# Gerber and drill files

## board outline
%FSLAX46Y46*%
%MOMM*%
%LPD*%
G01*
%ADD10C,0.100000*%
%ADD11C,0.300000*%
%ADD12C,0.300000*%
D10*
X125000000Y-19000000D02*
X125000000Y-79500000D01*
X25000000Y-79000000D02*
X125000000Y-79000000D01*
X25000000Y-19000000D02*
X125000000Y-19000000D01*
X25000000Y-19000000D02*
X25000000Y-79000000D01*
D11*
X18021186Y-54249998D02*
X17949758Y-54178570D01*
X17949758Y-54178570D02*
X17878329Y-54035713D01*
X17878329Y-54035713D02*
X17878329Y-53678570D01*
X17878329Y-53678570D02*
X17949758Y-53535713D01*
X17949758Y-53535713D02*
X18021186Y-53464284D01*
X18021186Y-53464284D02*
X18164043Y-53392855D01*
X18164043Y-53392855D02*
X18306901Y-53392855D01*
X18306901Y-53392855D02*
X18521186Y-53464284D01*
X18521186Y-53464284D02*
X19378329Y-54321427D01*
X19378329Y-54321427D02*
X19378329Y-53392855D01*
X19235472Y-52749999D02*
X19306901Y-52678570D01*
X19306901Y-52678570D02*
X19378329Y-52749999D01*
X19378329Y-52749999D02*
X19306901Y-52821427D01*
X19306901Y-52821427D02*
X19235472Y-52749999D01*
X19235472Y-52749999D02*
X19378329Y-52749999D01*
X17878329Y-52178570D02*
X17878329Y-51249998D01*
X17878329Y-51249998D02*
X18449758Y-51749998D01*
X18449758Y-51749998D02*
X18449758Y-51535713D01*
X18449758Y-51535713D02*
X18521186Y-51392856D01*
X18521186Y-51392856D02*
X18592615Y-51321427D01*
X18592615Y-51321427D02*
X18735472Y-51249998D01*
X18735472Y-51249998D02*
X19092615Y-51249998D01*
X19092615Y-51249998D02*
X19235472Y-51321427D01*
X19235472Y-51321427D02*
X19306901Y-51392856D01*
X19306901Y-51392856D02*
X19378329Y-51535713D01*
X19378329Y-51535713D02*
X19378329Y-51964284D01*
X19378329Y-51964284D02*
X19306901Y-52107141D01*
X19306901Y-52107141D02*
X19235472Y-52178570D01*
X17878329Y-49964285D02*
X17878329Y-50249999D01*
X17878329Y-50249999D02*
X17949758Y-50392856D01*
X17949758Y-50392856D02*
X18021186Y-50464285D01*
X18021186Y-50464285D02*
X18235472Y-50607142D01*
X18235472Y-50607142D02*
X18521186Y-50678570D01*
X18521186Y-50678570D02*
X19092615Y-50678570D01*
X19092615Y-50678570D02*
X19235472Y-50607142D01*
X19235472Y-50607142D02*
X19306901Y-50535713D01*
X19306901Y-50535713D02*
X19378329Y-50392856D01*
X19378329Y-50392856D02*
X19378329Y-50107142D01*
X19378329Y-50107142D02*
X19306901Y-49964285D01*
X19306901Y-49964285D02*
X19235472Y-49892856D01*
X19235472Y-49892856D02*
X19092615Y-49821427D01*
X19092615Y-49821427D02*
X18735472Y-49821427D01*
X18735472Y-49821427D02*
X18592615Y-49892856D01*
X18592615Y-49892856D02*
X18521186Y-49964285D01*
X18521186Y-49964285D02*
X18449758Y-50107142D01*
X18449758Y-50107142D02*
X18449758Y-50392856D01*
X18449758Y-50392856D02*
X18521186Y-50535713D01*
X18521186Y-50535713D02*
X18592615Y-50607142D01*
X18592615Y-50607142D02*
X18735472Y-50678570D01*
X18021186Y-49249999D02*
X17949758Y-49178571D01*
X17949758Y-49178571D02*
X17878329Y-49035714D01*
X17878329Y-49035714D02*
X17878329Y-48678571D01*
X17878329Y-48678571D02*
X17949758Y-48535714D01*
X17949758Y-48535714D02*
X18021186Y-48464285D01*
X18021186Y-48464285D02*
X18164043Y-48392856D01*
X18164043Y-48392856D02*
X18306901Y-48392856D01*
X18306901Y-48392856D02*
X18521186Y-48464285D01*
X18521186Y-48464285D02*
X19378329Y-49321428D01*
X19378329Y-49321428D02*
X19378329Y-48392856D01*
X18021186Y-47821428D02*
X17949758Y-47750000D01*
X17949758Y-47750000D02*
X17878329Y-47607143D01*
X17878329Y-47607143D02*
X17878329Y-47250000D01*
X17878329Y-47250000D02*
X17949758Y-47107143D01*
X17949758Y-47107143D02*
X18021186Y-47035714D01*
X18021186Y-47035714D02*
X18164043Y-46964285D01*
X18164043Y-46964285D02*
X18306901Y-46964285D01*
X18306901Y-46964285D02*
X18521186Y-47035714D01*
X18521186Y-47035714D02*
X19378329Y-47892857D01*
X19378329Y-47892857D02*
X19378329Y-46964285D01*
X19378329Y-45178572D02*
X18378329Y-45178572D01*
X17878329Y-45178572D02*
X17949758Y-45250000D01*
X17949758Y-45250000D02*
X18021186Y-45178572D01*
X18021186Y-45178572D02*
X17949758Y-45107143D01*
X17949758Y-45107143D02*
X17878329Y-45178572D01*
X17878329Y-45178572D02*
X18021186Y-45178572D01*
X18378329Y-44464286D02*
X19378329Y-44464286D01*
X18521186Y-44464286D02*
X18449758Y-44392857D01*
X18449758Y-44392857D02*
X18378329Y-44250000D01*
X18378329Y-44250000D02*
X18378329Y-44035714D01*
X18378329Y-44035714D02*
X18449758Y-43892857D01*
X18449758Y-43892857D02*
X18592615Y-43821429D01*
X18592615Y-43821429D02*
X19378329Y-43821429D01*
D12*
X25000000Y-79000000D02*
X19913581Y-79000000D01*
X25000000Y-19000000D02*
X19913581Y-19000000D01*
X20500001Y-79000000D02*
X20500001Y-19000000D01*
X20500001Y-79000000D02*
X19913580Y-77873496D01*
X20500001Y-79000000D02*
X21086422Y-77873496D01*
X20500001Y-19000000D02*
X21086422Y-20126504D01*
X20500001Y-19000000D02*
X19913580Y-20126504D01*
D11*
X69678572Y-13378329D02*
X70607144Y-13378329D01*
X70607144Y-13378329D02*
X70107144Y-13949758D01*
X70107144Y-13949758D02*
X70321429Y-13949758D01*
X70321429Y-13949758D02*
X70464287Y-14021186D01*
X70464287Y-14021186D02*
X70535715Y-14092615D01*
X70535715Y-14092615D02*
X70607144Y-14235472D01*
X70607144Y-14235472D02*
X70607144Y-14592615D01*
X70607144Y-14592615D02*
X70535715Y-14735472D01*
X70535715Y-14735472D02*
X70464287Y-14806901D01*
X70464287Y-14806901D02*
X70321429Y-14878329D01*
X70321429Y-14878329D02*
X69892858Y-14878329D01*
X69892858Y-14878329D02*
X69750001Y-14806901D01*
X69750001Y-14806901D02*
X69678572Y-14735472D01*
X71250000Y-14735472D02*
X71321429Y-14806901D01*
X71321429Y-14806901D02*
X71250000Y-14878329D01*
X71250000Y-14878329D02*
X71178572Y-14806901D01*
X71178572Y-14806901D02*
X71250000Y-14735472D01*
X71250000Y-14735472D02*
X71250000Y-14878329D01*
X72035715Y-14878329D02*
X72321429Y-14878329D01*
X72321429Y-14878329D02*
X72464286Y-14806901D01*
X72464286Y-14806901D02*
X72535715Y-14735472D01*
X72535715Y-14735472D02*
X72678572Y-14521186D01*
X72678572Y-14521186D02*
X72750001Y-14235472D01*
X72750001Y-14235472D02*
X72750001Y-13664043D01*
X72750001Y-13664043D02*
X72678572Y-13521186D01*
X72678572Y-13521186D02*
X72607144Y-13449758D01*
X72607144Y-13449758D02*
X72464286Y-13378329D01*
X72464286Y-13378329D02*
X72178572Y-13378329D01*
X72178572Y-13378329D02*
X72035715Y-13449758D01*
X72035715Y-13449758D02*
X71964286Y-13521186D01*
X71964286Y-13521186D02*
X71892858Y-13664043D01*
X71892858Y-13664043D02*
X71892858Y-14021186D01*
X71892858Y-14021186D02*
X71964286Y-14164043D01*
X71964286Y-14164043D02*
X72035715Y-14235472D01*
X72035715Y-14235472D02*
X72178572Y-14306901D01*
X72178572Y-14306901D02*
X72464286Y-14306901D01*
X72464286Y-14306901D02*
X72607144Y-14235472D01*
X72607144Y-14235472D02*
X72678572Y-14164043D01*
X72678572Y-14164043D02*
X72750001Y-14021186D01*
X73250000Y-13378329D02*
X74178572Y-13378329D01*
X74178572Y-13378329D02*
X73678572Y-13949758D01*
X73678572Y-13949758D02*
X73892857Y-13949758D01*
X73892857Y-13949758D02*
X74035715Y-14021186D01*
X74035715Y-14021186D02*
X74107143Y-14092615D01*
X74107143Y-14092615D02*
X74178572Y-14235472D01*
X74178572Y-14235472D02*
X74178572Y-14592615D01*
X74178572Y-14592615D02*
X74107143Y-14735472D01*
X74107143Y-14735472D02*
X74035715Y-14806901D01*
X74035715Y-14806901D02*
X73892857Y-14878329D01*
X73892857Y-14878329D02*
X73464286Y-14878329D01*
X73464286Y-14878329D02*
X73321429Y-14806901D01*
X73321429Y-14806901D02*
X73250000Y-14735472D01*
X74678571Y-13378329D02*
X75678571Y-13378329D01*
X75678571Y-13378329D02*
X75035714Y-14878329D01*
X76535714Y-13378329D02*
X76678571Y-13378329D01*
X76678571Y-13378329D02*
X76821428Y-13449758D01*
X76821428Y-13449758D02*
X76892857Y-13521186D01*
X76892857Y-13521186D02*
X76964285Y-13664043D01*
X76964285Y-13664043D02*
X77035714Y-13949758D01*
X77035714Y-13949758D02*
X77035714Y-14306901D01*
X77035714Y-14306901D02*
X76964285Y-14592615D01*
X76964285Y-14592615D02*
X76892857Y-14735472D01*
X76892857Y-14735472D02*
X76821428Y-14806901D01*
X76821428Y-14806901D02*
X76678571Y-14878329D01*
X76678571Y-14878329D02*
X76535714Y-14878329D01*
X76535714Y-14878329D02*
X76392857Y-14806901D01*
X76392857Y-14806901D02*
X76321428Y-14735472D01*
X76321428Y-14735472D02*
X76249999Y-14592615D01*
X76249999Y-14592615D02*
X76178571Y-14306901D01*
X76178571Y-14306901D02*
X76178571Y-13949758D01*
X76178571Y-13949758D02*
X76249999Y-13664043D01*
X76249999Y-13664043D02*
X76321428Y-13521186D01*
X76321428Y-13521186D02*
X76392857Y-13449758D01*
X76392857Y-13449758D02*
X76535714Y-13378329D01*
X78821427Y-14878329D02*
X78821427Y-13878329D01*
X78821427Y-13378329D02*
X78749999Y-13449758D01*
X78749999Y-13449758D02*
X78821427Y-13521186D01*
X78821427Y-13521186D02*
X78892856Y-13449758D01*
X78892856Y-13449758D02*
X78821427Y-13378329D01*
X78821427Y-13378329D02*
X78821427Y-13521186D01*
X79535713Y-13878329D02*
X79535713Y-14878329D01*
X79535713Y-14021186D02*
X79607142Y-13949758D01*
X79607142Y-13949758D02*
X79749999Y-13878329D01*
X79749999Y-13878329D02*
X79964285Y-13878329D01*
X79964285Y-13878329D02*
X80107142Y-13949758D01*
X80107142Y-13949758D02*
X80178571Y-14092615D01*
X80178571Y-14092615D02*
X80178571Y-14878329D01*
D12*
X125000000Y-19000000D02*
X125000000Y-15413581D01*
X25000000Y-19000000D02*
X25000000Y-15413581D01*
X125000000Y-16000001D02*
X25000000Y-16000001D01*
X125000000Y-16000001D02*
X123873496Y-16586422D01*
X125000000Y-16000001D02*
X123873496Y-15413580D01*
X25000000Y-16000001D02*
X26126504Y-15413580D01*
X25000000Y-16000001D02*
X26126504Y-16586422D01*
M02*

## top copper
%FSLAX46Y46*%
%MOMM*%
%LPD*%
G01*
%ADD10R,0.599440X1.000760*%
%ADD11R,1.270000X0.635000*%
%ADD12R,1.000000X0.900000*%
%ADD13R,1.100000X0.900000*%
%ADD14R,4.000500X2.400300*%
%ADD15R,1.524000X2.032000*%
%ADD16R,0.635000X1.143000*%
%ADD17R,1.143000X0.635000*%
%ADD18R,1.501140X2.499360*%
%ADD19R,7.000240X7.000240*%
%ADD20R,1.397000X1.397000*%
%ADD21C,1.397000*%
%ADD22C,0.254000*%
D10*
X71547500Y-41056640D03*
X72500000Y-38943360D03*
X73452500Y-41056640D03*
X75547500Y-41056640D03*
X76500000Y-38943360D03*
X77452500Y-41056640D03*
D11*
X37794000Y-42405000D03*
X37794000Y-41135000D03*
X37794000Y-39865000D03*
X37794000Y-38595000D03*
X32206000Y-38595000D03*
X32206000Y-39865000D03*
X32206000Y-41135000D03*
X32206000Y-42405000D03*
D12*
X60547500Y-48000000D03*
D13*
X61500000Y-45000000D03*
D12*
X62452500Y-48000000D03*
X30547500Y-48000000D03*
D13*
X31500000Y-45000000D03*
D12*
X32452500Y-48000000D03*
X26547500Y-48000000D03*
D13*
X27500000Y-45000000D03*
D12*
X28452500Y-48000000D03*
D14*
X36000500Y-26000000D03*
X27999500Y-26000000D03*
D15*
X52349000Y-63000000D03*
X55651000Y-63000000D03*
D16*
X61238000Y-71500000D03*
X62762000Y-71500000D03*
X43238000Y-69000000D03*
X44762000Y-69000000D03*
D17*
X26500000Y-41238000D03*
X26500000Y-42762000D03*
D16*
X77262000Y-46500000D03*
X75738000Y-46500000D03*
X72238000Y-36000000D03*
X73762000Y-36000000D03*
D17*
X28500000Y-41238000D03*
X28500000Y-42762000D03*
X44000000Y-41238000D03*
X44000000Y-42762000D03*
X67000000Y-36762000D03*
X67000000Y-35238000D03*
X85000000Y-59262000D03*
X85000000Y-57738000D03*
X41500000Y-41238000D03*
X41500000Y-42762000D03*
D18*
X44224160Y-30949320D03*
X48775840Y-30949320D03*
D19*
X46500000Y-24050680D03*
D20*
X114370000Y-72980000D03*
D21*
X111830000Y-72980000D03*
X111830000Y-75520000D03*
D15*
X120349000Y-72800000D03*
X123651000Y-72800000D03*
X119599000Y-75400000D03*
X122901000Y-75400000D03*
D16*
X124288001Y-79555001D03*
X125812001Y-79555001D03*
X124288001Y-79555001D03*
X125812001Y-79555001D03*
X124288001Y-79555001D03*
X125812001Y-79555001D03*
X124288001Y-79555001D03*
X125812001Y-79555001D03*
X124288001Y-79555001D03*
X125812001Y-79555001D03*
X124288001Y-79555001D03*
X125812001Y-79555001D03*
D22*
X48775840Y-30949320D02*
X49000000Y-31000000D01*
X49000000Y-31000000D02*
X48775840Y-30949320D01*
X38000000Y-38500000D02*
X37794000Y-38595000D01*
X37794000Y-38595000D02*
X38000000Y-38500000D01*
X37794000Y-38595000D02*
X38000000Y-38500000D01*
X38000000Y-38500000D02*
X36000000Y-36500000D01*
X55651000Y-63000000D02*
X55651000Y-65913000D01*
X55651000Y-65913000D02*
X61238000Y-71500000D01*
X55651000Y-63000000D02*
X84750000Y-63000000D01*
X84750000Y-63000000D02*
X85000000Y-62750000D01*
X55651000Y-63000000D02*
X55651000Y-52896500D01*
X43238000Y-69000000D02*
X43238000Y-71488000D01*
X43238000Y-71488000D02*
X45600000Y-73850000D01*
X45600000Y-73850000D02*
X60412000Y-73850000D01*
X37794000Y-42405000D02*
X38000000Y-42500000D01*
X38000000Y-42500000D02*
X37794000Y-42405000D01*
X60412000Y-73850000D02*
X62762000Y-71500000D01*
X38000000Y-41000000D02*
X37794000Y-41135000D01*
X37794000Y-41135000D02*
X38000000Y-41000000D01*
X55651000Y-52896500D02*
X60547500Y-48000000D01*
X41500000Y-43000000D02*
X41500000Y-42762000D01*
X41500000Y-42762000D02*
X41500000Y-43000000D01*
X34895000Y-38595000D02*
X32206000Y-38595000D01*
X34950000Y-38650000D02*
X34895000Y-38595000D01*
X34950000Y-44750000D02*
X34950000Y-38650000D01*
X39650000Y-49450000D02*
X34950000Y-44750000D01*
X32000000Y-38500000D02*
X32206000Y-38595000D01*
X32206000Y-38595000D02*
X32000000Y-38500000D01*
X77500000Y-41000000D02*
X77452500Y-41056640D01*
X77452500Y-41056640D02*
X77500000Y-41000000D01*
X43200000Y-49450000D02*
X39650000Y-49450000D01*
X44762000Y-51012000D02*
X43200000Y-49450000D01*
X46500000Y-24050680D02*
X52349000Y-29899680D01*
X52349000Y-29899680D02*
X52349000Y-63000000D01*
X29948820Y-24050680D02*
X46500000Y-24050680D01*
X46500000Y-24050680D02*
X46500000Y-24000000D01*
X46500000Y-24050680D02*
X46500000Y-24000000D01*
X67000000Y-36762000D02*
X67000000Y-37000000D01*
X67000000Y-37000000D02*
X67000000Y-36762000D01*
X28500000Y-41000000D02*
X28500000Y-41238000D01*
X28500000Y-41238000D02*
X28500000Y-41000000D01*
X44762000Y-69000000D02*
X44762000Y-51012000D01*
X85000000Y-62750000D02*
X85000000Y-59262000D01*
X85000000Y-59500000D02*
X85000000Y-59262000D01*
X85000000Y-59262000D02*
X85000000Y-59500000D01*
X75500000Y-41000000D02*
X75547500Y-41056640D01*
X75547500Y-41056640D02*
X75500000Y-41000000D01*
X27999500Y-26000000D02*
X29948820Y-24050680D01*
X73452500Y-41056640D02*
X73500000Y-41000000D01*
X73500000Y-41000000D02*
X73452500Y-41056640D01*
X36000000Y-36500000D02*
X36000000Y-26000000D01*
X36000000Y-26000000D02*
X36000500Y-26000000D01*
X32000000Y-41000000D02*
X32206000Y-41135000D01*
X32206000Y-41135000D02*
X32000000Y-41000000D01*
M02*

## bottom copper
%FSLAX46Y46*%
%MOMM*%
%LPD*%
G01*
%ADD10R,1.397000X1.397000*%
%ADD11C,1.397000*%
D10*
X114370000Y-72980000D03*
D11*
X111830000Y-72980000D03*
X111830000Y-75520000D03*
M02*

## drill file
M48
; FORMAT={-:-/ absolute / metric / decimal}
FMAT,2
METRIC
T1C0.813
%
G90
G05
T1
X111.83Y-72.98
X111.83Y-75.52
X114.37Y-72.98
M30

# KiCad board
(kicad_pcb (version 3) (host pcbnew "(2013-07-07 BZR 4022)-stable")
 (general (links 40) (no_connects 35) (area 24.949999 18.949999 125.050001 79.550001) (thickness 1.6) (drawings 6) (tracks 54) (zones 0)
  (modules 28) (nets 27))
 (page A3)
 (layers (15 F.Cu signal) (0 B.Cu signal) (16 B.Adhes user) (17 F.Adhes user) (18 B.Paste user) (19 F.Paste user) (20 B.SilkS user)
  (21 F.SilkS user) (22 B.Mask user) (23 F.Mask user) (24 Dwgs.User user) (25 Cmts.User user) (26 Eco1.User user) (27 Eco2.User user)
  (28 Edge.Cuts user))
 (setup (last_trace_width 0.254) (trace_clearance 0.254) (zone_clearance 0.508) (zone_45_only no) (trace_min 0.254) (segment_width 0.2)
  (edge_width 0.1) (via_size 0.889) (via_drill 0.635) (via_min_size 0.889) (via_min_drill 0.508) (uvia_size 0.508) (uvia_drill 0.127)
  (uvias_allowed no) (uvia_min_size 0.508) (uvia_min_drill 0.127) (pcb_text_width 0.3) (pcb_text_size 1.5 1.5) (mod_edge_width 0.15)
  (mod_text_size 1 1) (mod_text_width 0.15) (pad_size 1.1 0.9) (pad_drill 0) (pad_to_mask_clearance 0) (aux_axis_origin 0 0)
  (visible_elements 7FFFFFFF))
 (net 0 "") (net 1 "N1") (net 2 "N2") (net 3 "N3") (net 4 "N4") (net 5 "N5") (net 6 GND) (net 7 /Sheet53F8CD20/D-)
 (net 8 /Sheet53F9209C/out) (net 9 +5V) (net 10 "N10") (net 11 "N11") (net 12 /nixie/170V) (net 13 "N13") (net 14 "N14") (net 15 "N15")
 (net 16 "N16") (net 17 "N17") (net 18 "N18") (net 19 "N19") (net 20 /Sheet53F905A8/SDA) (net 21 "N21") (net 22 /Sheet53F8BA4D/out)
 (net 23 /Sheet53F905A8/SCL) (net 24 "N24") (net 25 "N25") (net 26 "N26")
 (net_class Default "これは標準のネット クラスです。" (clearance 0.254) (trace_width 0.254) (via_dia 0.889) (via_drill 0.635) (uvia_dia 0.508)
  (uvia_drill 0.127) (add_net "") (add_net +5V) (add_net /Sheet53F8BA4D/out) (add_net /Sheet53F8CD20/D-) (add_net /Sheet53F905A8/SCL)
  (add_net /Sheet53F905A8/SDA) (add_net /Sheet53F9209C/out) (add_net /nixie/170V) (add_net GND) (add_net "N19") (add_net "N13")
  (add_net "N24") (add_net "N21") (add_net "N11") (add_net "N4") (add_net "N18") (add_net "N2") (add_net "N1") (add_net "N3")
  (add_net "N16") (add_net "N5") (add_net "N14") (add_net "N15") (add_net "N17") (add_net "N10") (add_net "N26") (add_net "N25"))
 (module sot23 (layer F.Cu) (at 72.5 40)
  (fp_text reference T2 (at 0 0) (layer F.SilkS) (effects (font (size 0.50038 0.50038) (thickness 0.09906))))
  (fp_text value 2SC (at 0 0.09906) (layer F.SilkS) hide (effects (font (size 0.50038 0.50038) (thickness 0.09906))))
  (pad 1 smd rect (at -0.9525 1.05664) (size 0.59944 1.00076) (layers F.Cu F.Paste F.Mask) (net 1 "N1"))
  (pad 2 smd rect (at 0 -1.05664) (size 0.59944 1.00076) (layers F.Cu F.Paste F.Mask) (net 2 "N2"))
  (pad 3 smd rect (at 0.9525 1.05664) (size 0.59944 1.00076) (layers F.Cu F.Paste F.Mask) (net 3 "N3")))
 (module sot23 (layer F.Cu) (at 76.5 40)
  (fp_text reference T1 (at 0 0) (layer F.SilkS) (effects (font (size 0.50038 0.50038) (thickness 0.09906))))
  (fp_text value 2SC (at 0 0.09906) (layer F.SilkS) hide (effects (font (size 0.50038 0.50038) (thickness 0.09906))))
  (pad 1 smd rect (at -0.9525 1.05664) (size 0.59944 1.00076) (layers F.Cu F.Paste F.Mask) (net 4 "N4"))
  (pad 2 smd rect (at 0 -1.05664) (size 0.59944 1.00076) (layers F.Cu F.Paste F.Mask) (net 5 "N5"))
  (pad 3 smd rect (at 0.9525 1.05664) (size 0.59944 1.00076) (layers F.Cu F.Paste F.Mask) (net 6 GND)))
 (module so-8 (layer F.Cu) (at 35 40.5 90)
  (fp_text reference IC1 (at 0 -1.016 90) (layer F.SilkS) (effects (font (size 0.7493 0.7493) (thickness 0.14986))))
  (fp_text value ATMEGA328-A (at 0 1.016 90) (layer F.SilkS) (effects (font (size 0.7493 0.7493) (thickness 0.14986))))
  (pad 1 smd rect (at -1.905 2.794 90) (size 0.635 1.27) (layers F.Cu F.Paste F.Mask) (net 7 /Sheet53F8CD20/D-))
  (pad 2 smd rect (at -0.635 2.794 90) (size 0.635 1.27) (layers F.Cu F.Paste F.Mask) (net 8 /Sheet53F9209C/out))
  (pad 3 smd rect (at 0.635 2.794 90) (size 0.635 1.27) (layers F.Cu F.Paste F.Mask) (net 6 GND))
  (pad 4 smd rect (at 1.905 2.794 90) (size 0.635 1.27) (layers F.Cu F.Paste F.Mask) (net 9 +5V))
  (pad 5 smd rect (at 1.905 -2.794 90) (size 0.635 1.27) (layers F.Cu F.Paste F.Mask) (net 6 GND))
  (pad 6 smd rect (at 0.635 -2.794 90) (size 0.635 1.27) (layers F.Cu F.Paste F.Mask) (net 9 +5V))
  (pad 7 smd rect (at -0.635 -2.794 90) (size 0.635 1.27) (layers F.Cu F.Paste F.Mask) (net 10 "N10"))
  (pad 8 smd rect (at -1.905 -2.794 90) (size 0.635 1.27) (layers F.Cu F.Paste F.Mask) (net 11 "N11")))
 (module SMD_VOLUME (layer F.Cu) (at 61.5 46.5)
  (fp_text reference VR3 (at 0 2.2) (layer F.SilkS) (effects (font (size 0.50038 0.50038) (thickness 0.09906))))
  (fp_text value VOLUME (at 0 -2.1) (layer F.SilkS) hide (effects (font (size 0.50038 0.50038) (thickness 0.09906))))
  (pad 1 smd rect (at -0.9525 1.5) (size 1 0.9) (layers F.Cu F.Paste F.Mask) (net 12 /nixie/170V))
  (pad 2 smd rect (at 0 -1.5) (size 1.1 0.9) (layers F.Cu F.Paste F.Mask) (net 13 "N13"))
  (pad 3 smd rect (at 0.9525 1.5) (size 1 0.9) (layers F.Cu F.Paste F.Mask) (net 13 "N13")))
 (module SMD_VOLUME (layer F.Cu) (at 31.5 46.5)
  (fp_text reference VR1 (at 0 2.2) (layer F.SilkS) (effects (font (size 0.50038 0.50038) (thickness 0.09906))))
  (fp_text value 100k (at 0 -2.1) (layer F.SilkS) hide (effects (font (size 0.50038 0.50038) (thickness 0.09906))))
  (pad 1 smd rect (at -0.9525 1.5) (size 1 0.9) (layers F.Cu F.Paste F.Mask) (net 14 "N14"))
  (pad 2 smd rect (at 0 -1.5) (size 1.1 0.9) (layers F.Cu F.Paste F.Mask) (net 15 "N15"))
  (pad 3 smd rect (at 0.9525 1.5) (size 1 0.9) (layers F.Cu F.Paste F.Mask) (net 15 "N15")))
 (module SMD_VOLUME (layer F.Cu) (at 27.5 46.5)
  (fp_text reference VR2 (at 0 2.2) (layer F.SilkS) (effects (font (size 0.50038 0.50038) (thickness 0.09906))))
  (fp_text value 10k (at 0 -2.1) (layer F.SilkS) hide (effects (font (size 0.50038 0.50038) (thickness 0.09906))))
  (pad 1 smd rect (at -0.9525 1.5) (size 1 0.9) (layers F.Cu F.Paste F.Mask) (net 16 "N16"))
  (pad 2 smd rect (at 0 -1.5) (size 1.1 0.9) (layers F.Cu F.Paste F.Mask) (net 6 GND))
  (pad 3 smd rect (at 0.9525 1.5) (size 1 0.9) (layers F.Cu F.Paste F.Mask) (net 6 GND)))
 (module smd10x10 (layer F.Cu) (at 32 26)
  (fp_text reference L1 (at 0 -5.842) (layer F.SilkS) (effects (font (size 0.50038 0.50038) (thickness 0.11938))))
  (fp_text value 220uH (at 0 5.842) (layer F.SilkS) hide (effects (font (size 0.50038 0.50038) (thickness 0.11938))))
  (pad 1 smd rect (at 4.0005 0) (size 4.0005 2.4003) (layers F.Cu F.Paste F.Mask) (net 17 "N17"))
  (pad 2 smd rect (at -4.0005 0) (size 4.0005 2.4003) (layers F.Cu F.Paste F.Mask) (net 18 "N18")))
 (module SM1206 (layer F.Cu) (at 54 63)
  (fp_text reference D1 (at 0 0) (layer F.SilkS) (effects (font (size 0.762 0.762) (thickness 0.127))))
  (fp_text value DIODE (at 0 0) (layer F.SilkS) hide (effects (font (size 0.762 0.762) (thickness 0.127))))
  (pad 1 smd rect (at -1.651 0) (size 1.524 2.032) (layers F.Cu F.Paste F.Mask) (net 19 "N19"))
  (pad 2 smd rect (at 1.651 0) (size 1.524 2.032) (layers F.Cu F.Paste F.Mask) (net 9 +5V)))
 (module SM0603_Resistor (layer F.Cu) (at 62 71.5)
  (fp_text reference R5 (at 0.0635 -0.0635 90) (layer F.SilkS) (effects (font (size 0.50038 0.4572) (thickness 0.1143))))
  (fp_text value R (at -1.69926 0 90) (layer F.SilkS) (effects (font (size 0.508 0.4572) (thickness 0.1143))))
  (pad 1 smd rect (at -0.762 0) (size 0.635 1.143) (layers F.Cu F.Paste F.Mask) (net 9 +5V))
  (pad 2 smd rect (at 0.762 0) (size 0.635 1.143) (layers F.Cu F.Paste F.Mask) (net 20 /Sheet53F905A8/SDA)))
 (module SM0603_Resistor (layer F.Cu) (at 44 69)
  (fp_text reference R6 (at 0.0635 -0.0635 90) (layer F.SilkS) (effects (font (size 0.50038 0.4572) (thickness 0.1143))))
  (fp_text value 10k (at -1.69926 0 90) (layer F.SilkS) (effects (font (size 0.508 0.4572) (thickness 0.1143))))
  (pad 1 smd rect (at -0.762 0) (size 0.635 1.143) (layers F.Cu F.Paste F.Mask) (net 9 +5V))
  (pad 2 smd rect (at 0.762 0) (size 0.635 1.143) (layers F.Cu F.Paste F.Mask) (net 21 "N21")))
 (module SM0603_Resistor (layer F.Cu) (at 26.5 42 270)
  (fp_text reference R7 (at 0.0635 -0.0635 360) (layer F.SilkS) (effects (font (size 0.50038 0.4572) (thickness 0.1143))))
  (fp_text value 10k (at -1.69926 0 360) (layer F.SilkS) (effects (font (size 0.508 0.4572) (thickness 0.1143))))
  (pad 1 smd rect (at -0.762 0 270) (size 0.635 1.143) (layers F.Cu F.Paste F.Mask) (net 6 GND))
  (pad 2 smd rect (at 0.762 0 270) (size 0.635 1.143) (layers F.Cu F.Paste F.Mask) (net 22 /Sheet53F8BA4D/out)))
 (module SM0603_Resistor (layer F.Cu) (at 76.5 46.5 180)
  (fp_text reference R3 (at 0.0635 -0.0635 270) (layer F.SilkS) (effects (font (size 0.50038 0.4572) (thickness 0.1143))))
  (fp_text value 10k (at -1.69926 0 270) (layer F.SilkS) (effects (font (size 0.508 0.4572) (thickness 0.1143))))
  (pad 1 smd rect (at -0.762 0 180) (size 0.635 1.143) (layers F.Cu F.Paste F.Mask) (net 9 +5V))
  (pad 2 smd rect (at 0.762 0 180) (size 0.635 1.143) (layers F.Cu F.Paste F.Mask) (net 19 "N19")))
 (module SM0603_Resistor (layer F.Cu) (at 73 36)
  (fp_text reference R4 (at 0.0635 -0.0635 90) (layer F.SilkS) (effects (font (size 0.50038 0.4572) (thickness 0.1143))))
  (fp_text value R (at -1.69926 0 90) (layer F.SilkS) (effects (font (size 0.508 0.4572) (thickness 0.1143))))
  (pad 1 smd rect (at -0.762 0) (size 0.635 1.143) (layers F.Cu F.Paste F.Mask) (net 9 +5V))
  (pad 2 smd rect (at 0.762 0) (size 0.635 1.143) (layers F.Cu F.Paste F.Mask) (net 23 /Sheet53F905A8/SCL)))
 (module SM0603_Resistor (layer F.Cu) (at 28.5 42 270)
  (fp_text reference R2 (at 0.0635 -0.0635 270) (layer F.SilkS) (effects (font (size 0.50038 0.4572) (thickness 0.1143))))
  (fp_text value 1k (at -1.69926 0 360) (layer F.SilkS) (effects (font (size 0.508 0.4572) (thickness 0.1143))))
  (pad 1 smd rect (at -0.762 0 270) (size 0.635 1.143) (layers F.Cu F.Paste F.Mask) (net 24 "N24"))
  (pad 2 smd rect (at 0.762 0 270) (size 0.635 1.143) (layers F.Cu F.Paste F.Mask) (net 19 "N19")))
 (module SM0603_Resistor (layer F.Cu) (at 44 42 270)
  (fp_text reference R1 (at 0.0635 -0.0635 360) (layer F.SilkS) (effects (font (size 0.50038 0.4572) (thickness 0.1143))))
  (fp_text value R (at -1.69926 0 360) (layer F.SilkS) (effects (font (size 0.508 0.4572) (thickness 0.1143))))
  (pad 1 smd rect (at -0.762 0 270) (size 0.635 1.143) (layers F.Cu F.Paste F.Mask) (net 9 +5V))
  (pad 2 smd rect (at 0.762 0 270) (size 0.635 1.143) (layers F.Cu F.Paste F.Mask) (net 13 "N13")))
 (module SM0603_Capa (layer F.Cu) (at 67 36 90)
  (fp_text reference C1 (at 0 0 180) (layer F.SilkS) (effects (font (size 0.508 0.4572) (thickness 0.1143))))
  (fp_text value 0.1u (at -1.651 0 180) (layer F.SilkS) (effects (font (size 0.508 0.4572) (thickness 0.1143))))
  (pad 1 smd rect (at -0.762 0 90) (size 0.635 1.143) (layers F.Cu F.Paste F.Mask) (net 13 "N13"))
  (pad 2 smd rect (at 0.762 0 90) (size 0.635 1.143) (layers F.Cu F.Paste F.Mask) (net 6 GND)))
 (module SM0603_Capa (layer F.Cu) (at 85 58.5 90)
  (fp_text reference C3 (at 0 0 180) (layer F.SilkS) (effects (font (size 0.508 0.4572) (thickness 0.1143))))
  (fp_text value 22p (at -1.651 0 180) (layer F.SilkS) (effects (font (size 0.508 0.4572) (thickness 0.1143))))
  (pad 1 smd rect (at -0.762 0 90) (size 0.635 1.143) (layers F.Cu F.Paste F.Mask) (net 11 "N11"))
  (pad 2 smd rect (at 0.762 0 90) (size 0.635 1.143) (layers F.Cu F.Paste F.Mask) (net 6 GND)))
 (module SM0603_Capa (layer F.Cu) (at 41.5 42 270)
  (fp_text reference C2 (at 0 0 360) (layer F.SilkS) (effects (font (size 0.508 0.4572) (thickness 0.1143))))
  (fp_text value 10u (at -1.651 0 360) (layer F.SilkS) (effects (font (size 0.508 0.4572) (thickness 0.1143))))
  (pad 1 smd rect (at -0.762 0 270) (size 0.635 1.143) (layers F.Cu F.Paste F.Mask) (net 19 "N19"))
  (pad 2 smd rect (at 0.762 0 270) (size 0.635 1.143) (layers F.Cu F.Paste F.Mask) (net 6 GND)))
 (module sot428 (layer F.Cu) (at 46.5 27.5)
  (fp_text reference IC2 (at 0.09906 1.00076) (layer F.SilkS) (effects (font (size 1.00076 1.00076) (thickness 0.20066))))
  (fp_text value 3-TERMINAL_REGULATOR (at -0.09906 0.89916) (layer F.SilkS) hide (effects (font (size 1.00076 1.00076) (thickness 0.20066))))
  (pad 1 smd rect (at -2.27584 3.44932) (size 1.50114 2.49936) (layers F.Cu F.Paste F.Mask))
  (pad 3 smd rect (at 2.27584 3.44932) (size 1.50114 2.49936) (layers F.Cu F.Paste F.Mask))
  (pad 2 smd rect (at 0 -3.44932) (size 7.00024 7.00024) (layers F.Cu F.Paste F.Mask)))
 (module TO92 (layer F.Cu) (at 113.1 74.25)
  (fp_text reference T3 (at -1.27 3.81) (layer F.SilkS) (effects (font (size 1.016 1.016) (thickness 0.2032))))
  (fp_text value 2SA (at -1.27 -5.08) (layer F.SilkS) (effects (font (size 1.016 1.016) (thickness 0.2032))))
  (pad 1 thru_hole rect (at 1.27 -1.27) (size 1.397 1.397) (drill 0.8128) (layers *.Cu *.Mask F.SilkS) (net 1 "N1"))
  (pad 2 thru_hole circle (at -1.27 -1.27) (size 1.397 1.397) (drill 0.8128) (layers *.Cu *.Mask F.SilkS) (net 6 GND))
  (pad 3 thru_hole circle (at -1.27 1.27) (size 1.397 1.397) (drill 0.8128) (layers *.Cu *.Mask F.SilkS) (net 3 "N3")))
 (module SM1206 (layer F.Cu) (at 122 72.8)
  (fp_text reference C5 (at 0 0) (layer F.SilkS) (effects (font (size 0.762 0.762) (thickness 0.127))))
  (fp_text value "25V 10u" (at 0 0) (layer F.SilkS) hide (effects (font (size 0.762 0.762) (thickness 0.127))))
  (pad 1 smd rect (at -1.651 0) (size 1.524 2.032) (layers F.Cu F.Paste F.Mask) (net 17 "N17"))
  (pad 2 smd rect (at 1.651 0) (size 1.524 2.032) (layers F.Cu F.Paste F.Mask) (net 6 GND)))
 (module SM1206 (layer F.Cu) (at 121.25 75.4)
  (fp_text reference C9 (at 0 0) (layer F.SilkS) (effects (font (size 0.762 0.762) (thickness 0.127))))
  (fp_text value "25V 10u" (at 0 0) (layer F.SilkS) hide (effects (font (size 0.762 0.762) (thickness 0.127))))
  (pad 1 smd rect (at -1.651 0) (size 1.524 2.032) (layers F.Cu F.Paste F.Mask) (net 9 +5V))
  (pad 2 smd rect (at 1.651 0) (size 1.524 2.032) (layers F.Cu F.Paste F.Mask) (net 6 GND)))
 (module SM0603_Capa (layer F.Cu) (at 125.050001 79.555001)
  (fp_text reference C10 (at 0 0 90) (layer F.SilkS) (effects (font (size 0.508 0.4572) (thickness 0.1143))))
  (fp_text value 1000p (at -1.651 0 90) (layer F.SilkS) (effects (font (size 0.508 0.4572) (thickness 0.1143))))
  (pad 1 smd rect (at -0.762 0) (size 0.635 1.143) (layers F.Cu F.Paste F.Mask) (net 15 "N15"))
  (pad 2 smd rect (at 0.762 0) (size 0.635 1.143) (layers F.Cu F.Paste F.Mask) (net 6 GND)))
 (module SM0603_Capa (layer F.Cu) (at 125.050001 79.555001)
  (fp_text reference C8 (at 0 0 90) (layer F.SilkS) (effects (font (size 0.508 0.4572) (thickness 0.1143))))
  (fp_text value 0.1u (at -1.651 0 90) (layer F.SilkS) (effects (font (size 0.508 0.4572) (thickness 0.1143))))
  (pad 1 smd rect (at -0.762 0) (size 0.635 1.143) (layers F.Cu F.Paste F.Mask) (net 6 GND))
  (pad 2 smd rect (at 0.762 0) (size 0.635 1.143) (layers F.Cu F.Paste F.Mask) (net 17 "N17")))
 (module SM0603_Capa (layer F.Cu) (at 125.050001 79.555001)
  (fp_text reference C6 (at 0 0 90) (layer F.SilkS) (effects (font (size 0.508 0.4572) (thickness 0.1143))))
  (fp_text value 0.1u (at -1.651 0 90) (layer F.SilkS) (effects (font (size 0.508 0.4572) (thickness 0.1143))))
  (pad 1 smd rect (at -0.762 0) (size 0.635 1.143) (layers F.Cu F.Paste F.Mask) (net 17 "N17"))
  (pad 2 smd rect (at 0.762 0) (size 0.635 1.143) (layers F.Cu F.Paste F.Mask) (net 6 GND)))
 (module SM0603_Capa (layer F.Cu) (at 125.050001 79.555001)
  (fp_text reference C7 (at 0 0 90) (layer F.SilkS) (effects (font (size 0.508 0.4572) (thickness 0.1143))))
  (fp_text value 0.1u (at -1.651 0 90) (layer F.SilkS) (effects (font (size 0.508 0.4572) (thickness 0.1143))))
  (pad 1 smd rect (at -0.762 0) (size 0.635 1.143) (layers F.Cu F.Paste F.Mask) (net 9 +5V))
  (pad 2 smd rect (at 0.762 0) (size 0.635 1.143) (layers F.Cu F.Paste F.Mask) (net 6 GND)))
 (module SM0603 (layer F.Cu) (at 125.050001 79.555001)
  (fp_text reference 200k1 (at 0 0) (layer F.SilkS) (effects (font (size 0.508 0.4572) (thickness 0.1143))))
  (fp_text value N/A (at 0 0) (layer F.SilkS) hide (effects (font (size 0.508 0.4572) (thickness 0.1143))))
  (pad 1 smd rect (at -0.762 0) (size 0.635 1.143) (layers F.Cu F.Paste F.Mask) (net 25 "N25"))
  (pad 2 smd rect (at 0.762 0) (size 0.635 1.143) (layers F.Cu F.Paste F.Mask) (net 6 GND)))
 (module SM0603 (layer F.Cu) (at 125.050001 79.555001)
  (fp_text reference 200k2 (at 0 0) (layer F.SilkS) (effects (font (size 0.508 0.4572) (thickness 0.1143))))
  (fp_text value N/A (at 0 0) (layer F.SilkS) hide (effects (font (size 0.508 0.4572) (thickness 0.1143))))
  (pad 1 smd rect (at -0.762 0) (size 0.635 1.143) (layers F.Cu F.Paste F.Mask) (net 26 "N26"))
  (pad 2 smd rect (at 0.762 0) (size 0.635 1.143) (layers F.Cu F.Paste F.Mask) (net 6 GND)))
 (gr_line (start 125 19) (end 125 79.5) (angle 90) (layer Edge.Cuts) (width 0.1))
 (gr_line (start 25 79) (end 125 79) (angle 90) (layer Edge.Cuts) (width 0.1))
 (gr_line (start 25 19) (end 125 19) (angle 90) (layer Edge.Cuts) (width 0.1))
 (gr_line (start 25 19) (end 25 79) (angle 90) (layer Edge.Cuts) (width 0.1))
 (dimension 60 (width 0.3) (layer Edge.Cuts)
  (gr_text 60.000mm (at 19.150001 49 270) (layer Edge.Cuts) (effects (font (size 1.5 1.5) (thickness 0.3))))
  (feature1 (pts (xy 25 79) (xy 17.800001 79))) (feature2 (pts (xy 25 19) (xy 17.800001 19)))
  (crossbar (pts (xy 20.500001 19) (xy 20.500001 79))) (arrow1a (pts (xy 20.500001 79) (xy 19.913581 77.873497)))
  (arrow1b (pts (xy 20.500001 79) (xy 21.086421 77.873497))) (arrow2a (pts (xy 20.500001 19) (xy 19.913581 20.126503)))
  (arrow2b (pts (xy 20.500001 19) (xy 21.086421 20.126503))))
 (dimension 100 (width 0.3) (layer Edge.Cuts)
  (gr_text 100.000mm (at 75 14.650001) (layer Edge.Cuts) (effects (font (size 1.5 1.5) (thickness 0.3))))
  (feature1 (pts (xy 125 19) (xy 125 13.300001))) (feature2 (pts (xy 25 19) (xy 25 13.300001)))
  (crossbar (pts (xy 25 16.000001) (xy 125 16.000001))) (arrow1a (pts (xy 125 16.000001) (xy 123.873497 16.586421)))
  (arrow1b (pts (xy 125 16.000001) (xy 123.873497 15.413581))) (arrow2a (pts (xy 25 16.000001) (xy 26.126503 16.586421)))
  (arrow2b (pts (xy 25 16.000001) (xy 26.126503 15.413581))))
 (segment (start 48.77584 30.94932) (end 49 31) (width 0.254) (layer F.Cu) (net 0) (status 80000))
 (segment (start 49 31) (end 48.77584 30.94932) (width 0.254) (layer F.Cu) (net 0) (status 80000))
 (segment (start 38 38.5) (end 37.794 38.595) (width 0.254) (layer F.Cu) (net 9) (status 80000))
 (segment (start 37.794 38.595) (end 38 38.5) (width 0.254) (layer F.Cu) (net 9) (status 80000))
 (segment (start 37.794 38.595) (end 38 38.5) (width 0.254) (layer F.Cu) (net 9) (status 80000))
 (segment (start 38 38.5) (end 36 36.5) (width 0.254) (layer F.Cu) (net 9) (status 80000))
 (segment (start 55.651 63) (end 55.651 65.913) (width 0.254) (layer F.Cu) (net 9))
 (segment (start 55.651 65.913) (end 61.238 71.5) (width 0.254) (layer F.Cu) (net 9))
 (segment (start 55.651 63) (end 84.75 63) (width 0.254) (layer F.Cu) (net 9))
 (segment (start 84.75 63) (end 85 62.75) (width 0.254) (layer F.Cu) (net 9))
 (segment (start 55.651 63) (end 55.651 52.8965) (width 0.254) (layer F.Cu) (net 9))
 (segment (start 43.238 69) (end 43.238 71.488) (width 0.254) (layer F.Cu) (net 9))
 (segment (start 43.238 71.488) (end 45.6 73.85) (width 0.254) (layer F.Cu) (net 9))
 (segment (start 45.6 73.85) (end 60.412 73.85) (width 0.254) (layer F.Cu) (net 9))
 (segment (start 37.794 42.405) (end 38 42.5) (width 0.254) (layer F.Cu) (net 7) (status 80000))
 (segment (start 38 42.5) (end 37.794 42.405) (width 0.254) (layer F.Cu) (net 7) (status 80000))
 (segment (start 60.412 73.85) (end 62.762 71.5) (width 0.254) (layer F.Cu) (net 20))
 (segment (start 38 41) (end 37.794 41.135) (width 0.254) (layer F.Cu) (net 8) (status 80000))
 (segment (start 37.794 41.135) (end 38 41) (width 0.254) (layer F.Cu) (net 8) (status 80000))
 (segment (start 55.651 52.8965) (end 60.5475 48) (width 0.254) (layer F.Cu) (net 12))
 (segment (start 41.5 43) (end 41.5 42.762) (width 0.254) (layer F.Cu) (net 6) (status 80000))
 (segment (start 41.5 42.762) (end 41.5 43) (width 0.254) (layer F.Cu) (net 6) (status 80000))
 (segment (start 34.895 38.595) (end 32.206 38.595) (width 0.254) (layer F.Cu) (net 6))
 (segment (start 34.95 38.65) (end 34.895 38.595) (width 0.254) (layer F.Cu) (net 6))
 (segment (start 34.95 44.75) (end 34.95 38.65) (width 0.254) (layer F.Cu) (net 6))
 (segment (start 39.65 49.45) (end 34.95 44.75) (width 0.254) (layer F.Cu) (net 6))
 (segment (start 32 38.5) (end 32.206 38.595) (width 0.254) (layer F.Cu) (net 6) (status 80000))
 (segment (start 32.206 38.595) (end 32 38.5) (width 0.254) (layer F.Cu) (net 6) (status 80000))
 (segment (start 77.5 41) (end 77.4525 41.05664) (width 0.254) (layer F.Cu) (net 6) (status 80000))
 (segment (start 77.4525 41.05664) (end 77.5 41) (width 0.254) (layer F.Cu) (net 6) (status 80000))
 (segment (start 43.2 49.45) (end 39.65 49.45) (width 0.254) (layer F.Cu) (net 6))
 (segment (start 44.762 51.012) (end 43.2 49.45) (width 0.254) (layer F.Cu) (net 6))
 (segment (start 46.5 24.05068) (end 52.349 29.89968) (width 0.254) (layer F.Cu) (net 19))
 (segment (start 52.349 29.89968) (end 52.349 63) (width 0.254) (layer F.Cu) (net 19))
 (segment (start 29.94882 24.05068) (end 46.5 24.05068) (width 0.254) (layer F.Cu) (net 19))
 (segment (start 46.5 24.05068) (end 46.5 24) (width 0.254) (layer F.Cu) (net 19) (status 80000))
 (segment (start 46.5 24.05068) (end 46.5 24) (width 0.254) (layer F.Cu) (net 19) (status 80000))
 (segment (start 67 36.762) (end 67 37) (width 0.254) (layer F.Cu) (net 13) (status 80000))
 (segment (start 67 37) (end 67 36.762) (width 0.254) (layer F.Cu) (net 13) (status 80000))
 (segment (start 28.5 41) (end 28.5 41.238) (width 0.254) (layer F.Cu) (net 24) (status 80000))
 (segment (start 28.5 41.238) (end 28.5 41) (width 0.254) (layer F.Cu) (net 24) (status 80000))
 (segment (start 44.762 69) (end 44.762 51.012) (width 0.254) (layer F.Cu) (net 21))
 (segment (start 85 62.75) (end 85 59.262) (width 0.254) (layer F.Cu) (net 11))
 (segment (start 85 59.5) (end 85 59.262) (width 0.254) (layer F.Cu) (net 11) (status 80000))
 (segment (start 85 59.262) (end 85 59.5) (width 0.254) (layer F.Cu) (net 11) (status 80000))
 (segment (start 75.5 41) (end 75.5475 41.05664) (width 0.254) (layer F.Cu) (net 4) (status 80000))
 (segment (start 75.5475 41.05664) (end 75.5 41) (width 0.254) (layer F.Cu) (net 4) (status 80000))
 (segment (start 27.9995 26) (end 29.94882 24.05068) (width 0.254) (layer F.Cu) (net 18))
 (segment (start 73.4525 41.05664) (end 73.5 41) (width 0.254) (layer F.Cu) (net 3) (status 80000))
 (segment (start 73.5 41) (end 73.4525 41.05664) (width 0.254) (layer F.Cu) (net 3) (status 80000))
 (segment (start 36 36.5) (end 36 26) (width 0.254) (layer F.Cu) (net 17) (status 80000))
 (segment (start 36 26) (end 36.0005 26) (width 0.254) (layer F.Cu) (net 17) (status 80000))
 (segment (start 32 41) (end 32.206 41.135) (width 0.254) (layer F.Cu) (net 10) (status 80000))
 (segment (start 32.206 41.135) (end 32 41) (width 0.254) (layer F.Cu) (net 10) (status 80000)))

